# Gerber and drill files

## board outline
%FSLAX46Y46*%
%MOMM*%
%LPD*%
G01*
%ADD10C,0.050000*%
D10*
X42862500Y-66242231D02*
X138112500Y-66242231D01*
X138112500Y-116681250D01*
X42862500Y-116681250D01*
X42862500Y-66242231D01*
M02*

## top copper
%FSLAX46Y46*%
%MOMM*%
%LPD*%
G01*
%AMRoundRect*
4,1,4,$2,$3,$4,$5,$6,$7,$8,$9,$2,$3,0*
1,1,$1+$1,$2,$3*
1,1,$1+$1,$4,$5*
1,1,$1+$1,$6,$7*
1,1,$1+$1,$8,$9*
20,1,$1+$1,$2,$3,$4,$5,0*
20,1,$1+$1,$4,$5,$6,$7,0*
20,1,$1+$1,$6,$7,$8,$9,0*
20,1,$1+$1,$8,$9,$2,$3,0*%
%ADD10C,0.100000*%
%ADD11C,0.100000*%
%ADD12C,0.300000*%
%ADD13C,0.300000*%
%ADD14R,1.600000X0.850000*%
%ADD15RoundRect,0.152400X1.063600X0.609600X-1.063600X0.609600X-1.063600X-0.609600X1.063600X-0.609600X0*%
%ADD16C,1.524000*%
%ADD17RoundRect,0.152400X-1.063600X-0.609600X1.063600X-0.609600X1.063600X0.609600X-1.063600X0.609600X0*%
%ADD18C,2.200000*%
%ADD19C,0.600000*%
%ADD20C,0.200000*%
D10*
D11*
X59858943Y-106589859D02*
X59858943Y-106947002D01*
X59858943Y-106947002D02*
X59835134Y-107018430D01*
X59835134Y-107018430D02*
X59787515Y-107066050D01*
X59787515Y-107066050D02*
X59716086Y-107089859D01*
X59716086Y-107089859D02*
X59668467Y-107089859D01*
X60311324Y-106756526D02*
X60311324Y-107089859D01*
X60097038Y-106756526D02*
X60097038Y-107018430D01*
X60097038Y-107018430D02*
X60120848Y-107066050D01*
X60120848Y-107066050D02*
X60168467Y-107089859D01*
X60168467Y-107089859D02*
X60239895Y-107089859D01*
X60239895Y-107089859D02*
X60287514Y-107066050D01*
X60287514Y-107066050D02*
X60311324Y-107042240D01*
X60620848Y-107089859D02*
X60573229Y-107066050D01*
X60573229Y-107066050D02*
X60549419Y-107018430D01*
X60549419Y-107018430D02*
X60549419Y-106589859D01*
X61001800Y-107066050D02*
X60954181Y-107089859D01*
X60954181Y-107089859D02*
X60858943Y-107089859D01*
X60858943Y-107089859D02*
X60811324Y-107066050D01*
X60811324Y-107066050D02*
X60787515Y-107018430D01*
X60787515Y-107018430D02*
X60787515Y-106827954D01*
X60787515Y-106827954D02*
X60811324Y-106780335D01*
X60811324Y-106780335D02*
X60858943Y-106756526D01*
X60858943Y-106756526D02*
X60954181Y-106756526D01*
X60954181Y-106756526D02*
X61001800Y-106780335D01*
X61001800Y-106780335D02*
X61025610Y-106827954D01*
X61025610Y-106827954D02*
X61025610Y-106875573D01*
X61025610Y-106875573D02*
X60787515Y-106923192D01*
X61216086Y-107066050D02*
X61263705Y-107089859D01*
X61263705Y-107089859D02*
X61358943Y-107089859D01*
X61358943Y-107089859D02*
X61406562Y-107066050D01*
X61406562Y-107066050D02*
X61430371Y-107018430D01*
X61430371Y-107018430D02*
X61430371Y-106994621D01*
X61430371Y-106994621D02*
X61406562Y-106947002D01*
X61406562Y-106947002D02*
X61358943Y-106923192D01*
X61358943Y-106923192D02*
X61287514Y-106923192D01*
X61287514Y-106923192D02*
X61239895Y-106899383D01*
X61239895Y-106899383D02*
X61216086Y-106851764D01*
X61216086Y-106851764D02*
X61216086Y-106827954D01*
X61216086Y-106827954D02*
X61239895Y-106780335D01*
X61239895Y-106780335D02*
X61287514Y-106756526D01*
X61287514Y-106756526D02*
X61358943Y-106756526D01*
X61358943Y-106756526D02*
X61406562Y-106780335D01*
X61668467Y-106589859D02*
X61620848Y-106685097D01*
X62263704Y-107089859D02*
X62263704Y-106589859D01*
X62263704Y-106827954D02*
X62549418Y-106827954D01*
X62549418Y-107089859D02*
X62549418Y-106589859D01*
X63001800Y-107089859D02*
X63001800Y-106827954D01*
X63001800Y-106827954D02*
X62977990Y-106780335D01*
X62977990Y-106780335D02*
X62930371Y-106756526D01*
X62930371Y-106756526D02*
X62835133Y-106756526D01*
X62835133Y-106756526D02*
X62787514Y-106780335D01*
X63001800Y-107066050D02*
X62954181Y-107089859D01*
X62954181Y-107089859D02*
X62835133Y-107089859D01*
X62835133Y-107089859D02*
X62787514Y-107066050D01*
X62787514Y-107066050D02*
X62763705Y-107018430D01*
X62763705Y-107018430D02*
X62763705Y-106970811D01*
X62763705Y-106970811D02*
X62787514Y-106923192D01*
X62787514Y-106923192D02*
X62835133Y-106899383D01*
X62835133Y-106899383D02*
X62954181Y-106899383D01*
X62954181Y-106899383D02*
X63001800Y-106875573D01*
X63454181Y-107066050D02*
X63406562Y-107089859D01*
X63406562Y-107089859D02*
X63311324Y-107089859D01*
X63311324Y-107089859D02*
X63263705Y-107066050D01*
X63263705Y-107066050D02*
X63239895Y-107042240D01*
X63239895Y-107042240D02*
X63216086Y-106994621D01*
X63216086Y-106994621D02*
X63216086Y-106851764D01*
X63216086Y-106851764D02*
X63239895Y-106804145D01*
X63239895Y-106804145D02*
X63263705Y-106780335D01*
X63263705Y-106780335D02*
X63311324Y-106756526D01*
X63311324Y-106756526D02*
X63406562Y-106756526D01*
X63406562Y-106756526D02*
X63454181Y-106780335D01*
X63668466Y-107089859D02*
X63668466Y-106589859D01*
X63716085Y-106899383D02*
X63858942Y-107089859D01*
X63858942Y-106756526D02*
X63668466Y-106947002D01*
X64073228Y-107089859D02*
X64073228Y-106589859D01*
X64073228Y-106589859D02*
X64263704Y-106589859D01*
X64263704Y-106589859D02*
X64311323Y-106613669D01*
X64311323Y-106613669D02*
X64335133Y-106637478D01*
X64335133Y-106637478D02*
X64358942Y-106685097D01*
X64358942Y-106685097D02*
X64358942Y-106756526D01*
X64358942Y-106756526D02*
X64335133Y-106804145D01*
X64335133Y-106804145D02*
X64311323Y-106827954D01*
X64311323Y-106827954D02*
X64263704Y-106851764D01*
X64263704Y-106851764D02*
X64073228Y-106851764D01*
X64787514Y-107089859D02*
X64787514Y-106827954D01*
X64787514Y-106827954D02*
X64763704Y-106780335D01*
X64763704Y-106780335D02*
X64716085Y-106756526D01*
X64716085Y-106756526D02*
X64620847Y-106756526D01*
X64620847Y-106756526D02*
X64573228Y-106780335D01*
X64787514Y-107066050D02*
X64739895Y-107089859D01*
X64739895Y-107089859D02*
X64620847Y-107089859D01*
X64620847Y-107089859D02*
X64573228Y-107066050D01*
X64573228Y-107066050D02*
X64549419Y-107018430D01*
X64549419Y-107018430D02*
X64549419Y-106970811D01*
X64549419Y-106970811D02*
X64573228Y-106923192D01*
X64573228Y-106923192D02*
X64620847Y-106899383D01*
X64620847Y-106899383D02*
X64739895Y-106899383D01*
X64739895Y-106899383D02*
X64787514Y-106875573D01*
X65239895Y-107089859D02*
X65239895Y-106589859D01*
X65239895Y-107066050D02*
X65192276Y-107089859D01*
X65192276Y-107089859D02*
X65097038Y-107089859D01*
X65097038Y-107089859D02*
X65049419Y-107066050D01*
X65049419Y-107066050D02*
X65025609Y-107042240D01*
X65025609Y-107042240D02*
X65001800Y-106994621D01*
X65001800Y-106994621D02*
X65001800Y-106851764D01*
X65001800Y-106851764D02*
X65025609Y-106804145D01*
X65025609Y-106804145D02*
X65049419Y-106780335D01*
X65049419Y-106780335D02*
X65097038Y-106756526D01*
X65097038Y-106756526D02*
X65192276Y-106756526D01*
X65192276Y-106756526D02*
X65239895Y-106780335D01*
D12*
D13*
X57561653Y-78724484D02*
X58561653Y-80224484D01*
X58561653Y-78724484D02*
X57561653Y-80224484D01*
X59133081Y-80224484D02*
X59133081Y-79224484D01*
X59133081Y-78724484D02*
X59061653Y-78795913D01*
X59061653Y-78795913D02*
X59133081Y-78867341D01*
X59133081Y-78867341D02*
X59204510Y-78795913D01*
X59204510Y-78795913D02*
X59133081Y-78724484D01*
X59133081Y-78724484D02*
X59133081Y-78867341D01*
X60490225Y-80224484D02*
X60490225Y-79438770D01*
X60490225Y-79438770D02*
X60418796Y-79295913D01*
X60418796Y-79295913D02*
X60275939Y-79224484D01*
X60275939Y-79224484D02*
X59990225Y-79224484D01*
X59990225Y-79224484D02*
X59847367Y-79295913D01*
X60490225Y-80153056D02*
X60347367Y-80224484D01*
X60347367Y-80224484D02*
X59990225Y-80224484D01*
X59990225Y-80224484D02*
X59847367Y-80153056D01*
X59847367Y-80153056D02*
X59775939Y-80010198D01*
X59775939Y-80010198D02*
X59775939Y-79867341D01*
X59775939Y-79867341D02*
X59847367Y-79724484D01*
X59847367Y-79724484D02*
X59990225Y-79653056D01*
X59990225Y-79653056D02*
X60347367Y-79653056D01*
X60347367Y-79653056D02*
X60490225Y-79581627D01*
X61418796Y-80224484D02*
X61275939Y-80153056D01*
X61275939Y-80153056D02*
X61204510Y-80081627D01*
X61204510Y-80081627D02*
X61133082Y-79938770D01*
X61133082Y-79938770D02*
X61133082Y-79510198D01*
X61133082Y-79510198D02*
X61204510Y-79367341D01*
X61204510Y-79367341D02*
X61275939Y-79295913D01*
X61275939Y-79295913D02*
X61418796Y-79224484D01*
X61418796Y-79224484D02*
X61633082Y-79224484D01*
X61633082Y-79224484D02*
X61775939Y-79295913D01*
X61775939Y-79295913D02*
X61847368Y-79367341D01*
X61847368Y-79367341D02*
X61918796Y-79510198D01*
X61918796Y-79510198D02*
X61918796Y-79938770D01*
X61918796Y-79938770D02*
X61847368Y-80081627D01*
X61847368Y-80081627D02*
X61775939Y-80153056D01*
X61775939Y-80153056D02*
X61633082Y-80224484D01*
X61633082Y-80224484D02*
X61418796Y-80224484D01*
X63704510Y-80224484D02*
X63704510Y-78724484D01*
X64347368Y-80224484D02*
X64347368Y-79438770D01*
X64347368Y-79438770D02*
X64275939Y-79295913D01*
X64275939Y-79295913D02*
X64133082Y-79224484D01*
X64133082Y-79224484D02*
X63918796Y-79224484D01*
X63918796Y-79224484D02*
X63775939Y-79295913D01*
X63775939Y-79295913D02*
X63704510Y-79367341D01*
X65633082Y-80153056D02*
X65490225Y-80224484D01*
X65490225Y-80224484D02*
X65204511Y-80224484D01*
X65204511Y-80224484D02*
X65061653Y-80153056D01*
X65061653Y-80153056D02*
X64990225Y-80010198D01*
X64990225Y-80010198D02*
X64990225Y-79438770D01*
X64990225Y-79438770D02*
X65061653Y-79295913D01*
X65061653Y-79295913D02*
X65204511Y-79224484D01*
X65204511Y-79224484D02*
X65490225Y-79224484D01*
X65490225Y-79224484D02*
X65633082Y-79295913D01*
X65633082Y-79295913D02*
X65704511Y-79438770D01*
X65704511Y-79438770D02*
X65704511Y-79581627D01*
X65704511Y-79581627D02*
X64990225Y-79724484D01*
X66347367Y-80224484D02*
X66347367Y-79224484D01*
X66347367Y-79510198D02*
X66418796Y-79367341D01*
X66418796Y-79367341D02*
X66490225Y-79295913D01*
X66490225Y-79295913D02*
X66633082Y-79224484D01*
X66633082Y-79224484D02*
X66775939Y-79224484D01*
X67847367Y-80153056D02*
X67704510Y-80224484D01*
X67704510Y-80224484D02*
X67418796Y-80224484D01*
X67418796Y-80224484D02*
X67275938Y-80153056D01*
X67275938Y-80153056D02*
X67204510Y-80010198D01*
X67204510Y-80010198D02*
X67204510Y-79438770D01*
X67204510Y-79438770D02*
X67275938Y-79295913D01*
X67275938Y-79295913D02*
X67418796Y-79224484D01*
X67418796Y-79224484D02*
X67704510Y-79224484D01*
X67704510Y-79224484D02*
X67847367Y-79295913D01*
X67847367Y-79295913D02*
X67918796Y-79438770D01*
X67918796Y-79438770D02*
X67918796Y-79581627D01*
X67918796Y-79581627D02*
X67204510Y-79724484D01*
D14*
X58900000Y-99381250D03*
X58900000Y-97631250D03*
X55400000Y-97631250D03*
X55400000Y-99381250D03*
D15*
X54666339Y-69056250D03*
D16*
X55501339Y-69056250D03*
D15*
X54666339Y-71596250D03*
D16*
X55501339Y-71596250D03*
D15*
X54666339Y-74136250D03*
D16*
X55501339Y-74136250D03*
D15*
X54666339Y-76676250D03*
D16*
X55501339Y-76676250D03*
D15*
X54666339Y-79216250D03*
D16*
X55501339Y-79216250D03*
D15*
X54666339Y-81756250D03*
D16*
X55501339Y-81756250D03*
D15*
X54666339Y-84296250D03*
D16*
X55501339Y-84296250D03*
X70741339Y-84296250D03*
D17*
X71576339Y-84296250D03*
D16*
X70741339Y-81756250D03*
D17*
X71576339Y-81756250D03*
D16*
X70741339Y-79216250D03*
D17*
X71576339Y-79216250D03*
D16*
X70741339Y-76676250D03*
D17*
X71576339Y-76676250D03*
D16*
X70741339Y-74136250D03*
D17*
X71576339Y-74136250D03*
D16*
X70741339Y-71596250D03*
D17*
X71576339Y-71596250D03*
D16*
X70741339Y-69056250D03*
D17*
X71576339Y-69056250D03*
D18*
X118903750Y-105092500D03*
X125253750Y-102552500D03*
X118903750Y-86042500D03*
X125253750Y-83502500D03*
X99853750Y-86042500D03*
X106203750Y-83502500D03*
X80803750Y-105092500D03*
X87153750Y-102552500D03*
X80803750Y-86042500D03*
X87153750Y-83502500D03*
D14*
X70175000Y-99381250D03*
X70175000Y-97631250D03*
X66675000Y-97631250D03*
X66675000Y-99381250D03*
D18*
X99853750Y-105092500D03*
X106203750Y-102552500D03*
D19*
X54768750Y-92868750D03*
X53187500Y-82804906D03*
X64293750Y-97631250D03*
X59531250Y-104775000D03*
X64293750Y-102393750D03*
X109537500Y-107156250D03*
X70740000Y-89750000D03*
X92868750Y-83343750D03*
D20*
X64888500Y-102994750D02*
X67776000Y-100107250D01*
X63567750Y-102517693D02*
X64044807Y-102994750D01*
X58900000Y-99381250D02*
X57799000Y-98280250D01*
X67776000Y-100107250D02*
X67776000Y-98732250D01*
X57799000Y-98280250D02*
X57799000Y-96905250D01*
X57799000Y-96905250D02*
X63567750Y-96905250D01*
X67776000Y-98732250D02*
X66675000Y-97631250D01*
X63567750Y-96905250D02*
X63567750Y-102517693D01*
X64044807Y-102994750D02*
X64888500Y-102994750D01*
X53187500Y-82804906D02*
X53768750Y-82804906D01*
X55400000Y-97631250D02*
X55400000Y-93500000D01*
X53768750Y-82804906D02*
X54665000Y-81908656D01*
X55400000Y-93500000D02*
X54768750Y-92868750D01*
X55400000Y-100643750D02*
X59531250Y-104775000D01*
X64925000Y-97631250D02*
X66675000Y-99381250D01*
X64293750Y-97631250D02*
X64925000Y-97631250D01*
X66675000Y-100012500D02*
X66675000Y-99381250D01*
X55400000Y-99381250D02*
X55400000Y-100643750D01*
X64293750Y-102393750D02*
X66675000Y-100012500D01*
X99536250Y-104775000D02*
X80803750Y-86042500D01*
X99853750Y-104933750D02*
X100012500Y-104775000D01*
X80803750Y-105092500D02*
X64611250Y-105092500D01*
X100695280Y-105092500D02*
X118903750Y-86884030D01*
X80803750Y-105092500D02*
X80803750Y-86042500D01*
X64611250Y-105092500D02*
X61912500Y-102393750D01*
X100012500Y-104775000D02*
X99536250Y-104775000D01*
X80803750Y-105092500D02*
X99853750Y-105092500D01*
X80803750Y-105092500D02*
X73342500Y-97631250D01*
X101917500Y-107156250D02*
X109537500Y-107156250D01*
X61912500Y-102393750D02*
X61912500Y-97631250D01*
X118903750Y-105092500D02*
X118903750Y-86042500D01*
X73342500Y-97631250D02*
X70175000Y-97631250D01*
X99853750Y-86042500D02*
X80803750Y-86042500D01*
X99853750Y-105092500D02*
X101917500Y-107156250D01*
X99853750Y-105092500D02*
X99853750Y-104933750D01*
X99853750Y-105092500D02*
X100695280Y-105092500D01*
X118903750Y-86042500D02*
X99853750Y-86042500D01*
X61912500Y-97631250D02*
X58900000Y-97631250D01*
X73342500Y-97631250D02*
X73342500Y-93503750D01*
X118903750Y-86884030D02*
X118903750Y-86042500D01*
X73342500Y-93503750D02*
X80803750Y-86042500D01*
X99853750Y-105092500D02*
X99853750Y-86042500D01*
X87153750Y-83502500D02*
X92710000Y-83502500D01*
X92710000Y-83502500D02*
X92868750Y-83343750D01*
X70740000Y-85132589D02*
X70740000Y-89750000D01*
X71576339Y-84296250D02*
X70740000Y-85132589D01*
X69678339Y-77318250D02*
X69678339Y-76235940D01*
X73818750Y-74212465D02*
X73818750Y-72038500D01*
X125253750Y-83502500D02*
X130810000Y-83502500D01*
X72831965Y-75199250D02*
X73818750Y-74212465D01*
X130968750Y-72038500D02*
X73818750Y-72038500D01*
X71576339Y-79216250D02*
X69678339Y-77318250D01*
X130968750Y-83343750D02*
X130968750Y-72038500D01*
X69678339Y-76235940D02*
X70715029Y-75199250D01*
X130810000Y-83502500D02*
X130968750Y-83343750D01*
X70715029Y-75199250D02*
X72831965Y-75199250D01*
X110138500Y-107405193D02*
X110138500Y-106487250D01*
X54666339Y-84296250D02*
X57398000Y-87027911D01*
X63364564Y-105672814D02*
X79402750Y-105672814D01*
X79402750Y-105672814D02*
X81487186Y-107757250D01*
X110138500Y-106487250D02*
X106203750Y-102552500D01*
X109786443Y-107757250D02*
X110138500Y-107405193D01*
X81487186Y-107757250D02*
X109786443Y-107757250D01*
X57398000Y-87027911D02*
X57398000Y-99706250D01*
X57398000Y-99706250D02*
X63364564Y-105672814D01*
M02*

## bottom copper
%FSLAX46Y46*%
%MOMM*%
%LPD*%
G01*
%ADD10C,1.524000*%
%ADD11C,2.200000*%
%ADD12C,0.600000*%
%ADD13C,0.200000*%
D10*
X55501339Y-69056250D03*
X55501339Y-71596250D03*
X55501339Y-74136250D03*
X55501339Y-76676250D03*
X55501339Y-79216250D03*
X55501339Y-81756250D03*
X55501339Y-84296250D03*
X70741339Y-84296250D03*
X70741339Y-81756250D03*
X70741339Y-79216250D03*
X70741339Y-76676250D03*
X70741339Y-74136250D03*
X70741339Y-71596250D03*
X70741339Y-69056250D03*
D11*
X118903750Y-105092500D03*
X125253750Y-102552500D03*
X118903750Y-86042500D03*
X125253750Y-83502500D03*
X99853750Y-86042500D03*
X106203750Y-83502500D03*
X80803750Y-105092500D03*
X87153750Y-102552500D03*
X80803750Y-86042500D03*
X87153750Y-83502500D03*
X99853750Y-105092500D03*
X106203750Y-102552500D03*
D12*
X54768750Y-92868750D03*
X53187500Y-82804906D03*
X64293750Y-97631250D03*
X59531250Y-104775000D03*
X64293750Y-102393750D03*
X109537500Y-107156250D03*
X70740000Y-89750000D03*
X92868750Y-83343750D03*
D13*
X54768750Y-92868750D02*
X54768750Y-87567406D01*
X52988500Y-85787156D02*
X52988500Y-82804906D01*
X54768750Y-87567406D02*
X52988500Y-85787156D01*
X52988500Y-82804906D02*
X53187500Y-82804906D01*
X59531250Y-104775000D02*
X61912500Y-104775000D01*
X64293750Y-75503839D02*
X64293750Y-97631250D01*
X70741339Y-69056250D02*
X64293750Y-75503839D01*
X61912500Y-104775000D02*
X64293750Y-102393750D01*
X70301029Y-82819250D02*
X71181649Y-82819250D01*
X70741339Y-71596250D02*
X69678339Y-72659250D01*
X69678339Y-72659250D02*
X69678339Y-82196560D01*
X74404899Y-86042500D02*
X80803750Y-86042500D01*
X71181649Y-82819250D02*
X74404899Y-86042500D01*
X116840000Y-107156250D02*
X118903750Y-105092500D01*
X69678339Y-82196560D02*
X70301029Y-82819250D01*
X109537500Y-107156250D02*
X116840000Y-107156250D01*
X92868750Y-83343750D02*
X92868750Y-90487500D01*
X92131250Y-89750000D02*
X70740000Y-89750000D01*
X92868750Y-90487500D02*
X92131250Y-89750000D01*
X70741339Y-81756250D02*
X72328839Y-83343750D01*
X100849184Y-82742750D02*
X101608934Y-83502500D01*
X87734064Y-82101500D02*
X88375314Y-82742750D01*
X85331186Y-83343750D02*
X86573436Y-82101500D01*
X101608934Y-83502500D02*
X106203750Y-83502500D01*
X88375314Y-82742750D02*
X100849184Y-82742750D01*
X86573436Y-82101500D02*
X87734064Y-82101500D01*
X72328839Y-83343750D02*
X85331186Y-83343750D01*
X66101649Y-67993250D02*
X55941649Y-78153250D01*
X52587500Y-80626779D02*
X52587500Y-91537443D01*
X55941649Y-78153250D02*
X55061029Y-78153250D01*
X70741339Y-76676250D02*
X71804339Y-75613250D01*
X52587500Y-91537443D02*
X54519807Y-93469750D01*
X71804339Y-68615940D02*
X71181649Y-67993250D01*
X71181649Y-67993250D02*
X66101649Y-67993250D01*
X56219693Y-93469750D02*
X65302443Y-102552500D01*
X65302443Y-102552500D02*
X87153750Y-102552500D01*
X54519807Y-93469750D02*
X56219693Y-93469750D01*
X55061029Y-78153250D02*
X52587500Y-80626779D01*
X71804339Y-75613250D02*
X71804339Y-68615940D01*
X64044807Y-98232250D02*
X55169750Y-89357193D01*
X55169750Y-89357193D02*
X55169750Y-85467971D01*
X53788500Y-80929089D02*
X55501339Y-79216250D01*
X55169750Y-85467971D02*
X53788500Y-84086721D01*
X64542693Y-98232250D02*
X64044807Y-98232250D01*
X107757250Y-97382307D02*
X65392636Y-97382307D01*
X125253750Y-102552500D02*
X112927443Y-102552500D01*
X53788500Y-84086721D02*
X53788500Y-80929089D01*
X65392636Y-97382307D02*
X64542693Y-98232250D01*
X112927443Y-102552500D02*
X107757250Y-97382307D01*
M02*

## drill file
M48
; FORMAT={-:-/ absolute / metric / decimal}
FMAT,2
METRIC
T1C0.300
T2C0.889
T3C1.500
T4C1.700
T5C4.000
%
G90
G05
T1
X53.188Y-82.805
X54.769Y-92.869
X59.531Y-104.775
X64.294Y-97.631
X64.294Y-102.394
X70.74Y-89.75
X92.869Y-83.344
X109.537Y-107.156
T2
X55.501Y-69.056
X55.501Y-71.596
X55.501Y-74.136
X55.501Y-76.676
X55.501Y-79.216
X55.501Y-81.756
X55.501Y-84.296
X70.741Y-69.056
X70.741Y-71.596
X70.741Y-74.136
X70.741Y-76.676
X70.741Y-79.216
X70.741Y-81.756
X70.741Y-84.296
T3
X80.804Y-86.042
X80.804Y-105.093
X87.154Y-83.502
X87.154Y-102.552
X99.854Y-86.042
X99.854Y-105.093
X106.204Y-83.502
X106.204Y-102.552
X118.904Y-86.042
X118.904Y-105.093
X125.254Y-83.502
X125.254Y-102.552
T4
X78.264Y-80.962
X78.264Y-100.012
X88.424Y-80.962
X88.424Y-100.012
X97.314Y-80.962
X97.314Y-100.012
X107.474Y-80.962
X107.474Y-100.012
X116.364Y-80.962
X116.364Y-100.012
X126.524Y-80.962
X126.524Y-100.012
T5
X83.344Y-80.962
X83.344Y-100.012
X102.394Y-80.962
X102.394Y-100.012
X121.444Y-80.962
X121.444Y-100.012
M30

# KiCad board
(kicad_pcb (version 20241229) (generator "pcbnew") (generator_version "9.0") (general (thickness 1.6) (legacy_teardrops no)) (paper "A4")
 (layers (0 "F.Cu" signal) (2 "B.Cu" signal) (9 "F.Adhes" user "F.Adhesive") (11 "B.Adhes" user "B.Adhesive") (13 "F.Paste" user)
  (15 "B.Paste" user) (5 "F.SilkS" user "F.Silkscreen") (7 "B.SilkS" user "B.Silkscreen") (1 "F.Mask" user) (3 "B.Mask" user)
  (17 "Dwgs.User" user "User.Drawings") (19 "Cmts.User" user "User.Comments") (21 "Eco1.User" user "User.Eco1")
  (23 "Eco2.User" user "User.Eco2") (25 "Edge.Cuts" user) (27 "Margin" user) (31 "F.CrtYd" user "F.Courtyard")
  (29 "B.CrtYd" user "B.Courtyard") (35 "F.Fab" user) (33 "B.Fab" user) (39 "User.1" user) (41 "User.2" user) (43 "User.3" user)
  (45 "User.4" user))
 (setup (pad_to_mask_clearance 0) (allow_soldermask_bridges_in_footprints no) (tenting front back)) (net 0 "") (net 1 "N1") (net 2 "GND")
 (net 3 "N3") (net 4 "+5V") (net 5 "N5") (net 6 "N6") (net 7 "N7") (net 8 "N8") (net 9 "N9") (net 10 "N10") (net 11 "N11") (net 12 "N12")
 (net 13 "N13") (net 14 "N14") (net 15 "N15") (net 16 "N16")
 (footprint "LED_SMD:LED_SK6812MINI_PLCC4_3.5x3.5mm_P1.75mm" (layer "F.Cu") (at 57.15 98.50625 180)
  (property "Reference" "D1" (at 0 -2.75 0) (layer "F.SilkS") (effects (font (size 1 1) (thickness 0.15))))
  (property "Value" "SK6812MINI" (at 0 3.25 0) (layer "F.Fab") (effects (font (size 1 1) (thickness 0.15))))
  (pad "1" smd rect (at -1.75 -0.875 180) (size 1.6 0.85) (layers "F.Cu" "F.Mask" "F.Paste") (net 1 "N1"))
  (pad "2" smd rect (at -1.75 0.875 180) (size 1.6 0.85) (layers "F.Cu" "F.Mask" "F.Paste") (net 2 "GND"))
  (pad "3" smd rect (at 1.75 0.875 180) (size 1.6 0.85) (layers "F.Cu" "F.Mask" "F.Paste") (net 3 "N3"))
  (pad "4" smd rect (at 1.75 -0.875 180) (size 1.6 0.85) (layers "F.Cu" "F.Mask" "F.Paste") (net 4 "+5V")))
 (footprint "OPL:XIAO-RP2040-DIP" (layer "F.Cu") (at 63.121339 76.67625)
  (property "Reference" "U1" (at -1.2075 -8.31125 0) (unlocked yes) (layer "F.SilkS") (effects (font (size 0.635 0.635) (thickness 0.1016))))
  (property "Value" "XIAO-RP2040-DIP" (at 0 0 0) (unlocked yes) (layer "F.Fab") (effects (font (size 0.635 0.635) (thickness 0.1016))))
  (pad "1" smd roundrect (at -8.455 -7.62 180) (size 2.432 1.524) (layers "F.Cu" "F.Mask") (roundrect_rratio 0.1) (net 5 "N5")
   (thermal_bridge_angle 45))
  (pad "1" thru_hole circle (at -7.62 -7.62 180) (size 1.524 1.524) (drill 0.889) (layers "*.Cu" "*.Mask") (remove_unused_layers no)
   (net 5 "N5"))
  (pad "2" smd roundrect (at -8.455 -5.08 180) (size 2.432 1.524) (layers "F.Cu" "F.Mask") (roundrect_rratio 0.1) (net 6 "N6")
   (thermal_bridge_angle 45))
  (pad "2" thru_hole circle (at -7.62 -5.08 180) (size 1.524 1.524) (drill 0.889) (layers "*.Cu" "*.Mask") (remove_unused_layers no)
   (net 6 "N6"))
  (pad "3" smd roundrect (at -8.455 -2.54 180) (size 2.432 1.524) (layers "F.Cu" "F.Mask") (roundrect_rratio 0.1) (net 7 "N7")
   (thermal_bridge_angle 45))
  (pad "3" thru_hole circle (at -7.62 -2.54 180) (size 1.524 1.524) (drill 0.889) (layers "*.Cu" "*.Mask") (remove_unused_layers no)
   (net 7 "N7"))
  (pad "4" smd roundrect (at -8.455 0 180) (size 2.432 1.524) (layers "F.Cu" "F.Mask") (roundrect_rratio 0.1) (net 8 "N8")
   (thermal_bridge_angle 45))
  (pad "4" thru_hole circle (at -7.62 0 180) (size 1.524 1.524) (drill 0.889) (layers "*.Cu" "*.Mask") (remove_unused_layers no)
   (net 8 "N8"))
  (pad "5" smd roundrect (at -8.455 2.54 180) (size 2.432 1.524) (layers "F.Cu" "F.Mask") (roundrect_rratio 0.1) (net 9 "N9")
   (thermal_bridge_angle 45))
  (pad "5" thru_hole circle (at -7.62 2.54 180) (size 1.524 1.524) (drill 0.889) (layers "*.Cu" "*.Mask") (remove_unused_layers no)
   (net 9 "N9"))
  (pad "6" smd roundrect (at -8.455 5.08 180) (size 2.432 1.524) (layers "F.Cu" "F.Mask") (roundrect_rratio 0.1) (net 3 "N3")
   (thermal_bridge_angle 45))
  (pad "6" thru_hole circle (at -7.62 5.08 180) (size 1.524 1.524) (drill 0.889) (layers "*.Cu" "*.Mask") (remove_unused_layers no)
   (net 3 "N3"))
  (pad "7" smd roundrect (at -8.455 7.62 180) (size 2.432 1.524) (layers "F.Cu" "F.Mask") (roundrect_rratio 0.1) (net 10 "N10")
   (thermal_bridge_angle 45))
  (pad "7" thru_hole circle (at -7.62 7.62 180) (size 1.524 1.524) (drill 0.889) (layers "*.Cu" "*.Mask") (remove_unused_layers no)
   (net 10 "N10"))
  (pad "8" thru_hole circle (at 7.62 7.62) (size 1.524 1.524) (drill 0.889) (layers "*.Cu" "*.Mask") (remove_unused_layers no)
   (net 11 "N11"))
  (pad "8" smd roundrect (at 8.455 7.62) (size 2.432 1.524) (layers "F.Cu" "F.Mask") (roundrect_rratio 0.1) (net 11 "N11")
   (thermal_bridge_angle 45))
  (pad "9" thru_hole circle (at 7.62 5.08) (size 1.524 1.524) (drill 0.889) (layers "*.Cu" "*.Mask") (remove_unused_layers no)
   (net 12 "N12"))
  (pad "9" smd roundrect (at 8.455 5.08) (size 2.432 1.524) (layers "F.Cu" "F.Mask") (roundrect_rratio 0.1) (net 12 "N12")
   (thermal_bridge_angle 45))
  (pad "10" thru_hole circle (at 7.62 2.54) (size 1.524 1.524) (drill 0.889) (layers "*.Cu" "*.Mask") (remove_unused_layers no)
   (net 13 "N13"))
  (pad "10" smd roundrect (at 8.455 2.54) (size 2.432 1.524) (layers "F.Cu" "F.Mask") (roundrect_rratio 0.1) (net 13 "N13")
   (thermal_bridge_angle 45))
  (pad "11" thru_hole circle (at 7.62 0) (size 1.524 1.524) (drill 0.889) (layers "*.Cu" "*.Mask") (remove_unused_layers no) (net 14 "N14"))
  (pad "11" smd roundrect (at 8.455 0) (size 2.432 1.524) (layers "F.Cu" "F.Mask") (roundrect_rratio 0.1) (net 14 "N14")
   (thermal_bridge_angle 45))
  (pad "12" thru_hole circle (at 7.62 -2.54) (size 1.524 1.524) (drill 0.889) (layers "*.Cu" "*.Mask") (remove_unused_layers no)
   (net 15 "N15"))
  (pad "12" smd roundrect (at 8.455 -2.54) (size 2.432 1.524) (layers "F.Cu" "F.Mask") (roundrect_rratio 0.1) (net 15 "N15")
   (thermal_bridge_angle 45))
  (pad "13" thru_hole circle (at 7.62 -5.08) (size 1.524 1.524) (drill 0.889) (layers "*.Cu" "*.Mask") (remove_unused_layers no)
   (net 2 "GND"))
  (pad "13" smd roundrect (at 8.455 -5.08) (size 2.432 1.524) (layers "F.Cu" "F.Mask") (roundrect_rratio 0.1) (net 2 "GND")
   (thermal_bridge_angle 45))
  (pad "14" thru_hole circle (at 7.62 -7.62) (size 1.524 1.524) (drill 0.889) (layers "*.Cu" "*.Mask") (remove_unused_layers no)
   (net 4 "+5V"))
  (pad "14" smd roundrect (at 8.455 -7.62) (size 2.432 1.524) (layers "F.Cu" "F.Mask") (roundrect_rratio 0.1) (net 4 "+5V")
   (thermal_bridge_angle 45)))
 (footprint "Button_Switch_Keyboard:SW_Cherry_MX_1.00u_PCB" (layer "F.Cu") (at 118.90375 105.0925 180)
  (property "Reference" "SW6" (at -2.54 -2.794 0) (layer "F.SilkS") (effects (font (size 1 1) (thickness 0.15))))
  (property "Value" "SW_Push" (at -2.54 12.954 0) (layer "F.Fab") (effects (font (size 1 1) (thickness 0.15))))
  (pad "" np_thru_hole circle (at -7.62 5.08 180) (size 1.7 1.7) (drill 1.7) (layers "*.Cu" "*.Mask"))
  (pad "" np_thru_hole circle (at -2.54 5.08 180) (size 4 4) (drill 4) (layers "*.Cu" "*.Mask"))
  (pad "" np_thru_hole circle (at 2.54 5.08 180) (size 1.7 1.7) (drill 1.7) (layers "*.Cu" "*.Mask"))
  (pad "1" thru_hole circle (at 0 0 180) (size 2.2 2.2) (drill 1.5) (layers "*.Cu" "*.Mask") (remove_unused_layers no) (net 2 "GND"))
  (pad "2" thru_hole circle (at -6.35 2.54 180) (size 2.2 2.2) (drill 1.5) (layers "*.Cu" "*.Mask") (remove_unused_layers no) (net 9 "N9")))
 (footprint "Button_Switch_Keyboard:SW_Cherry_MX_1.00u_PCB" (layer "F.Cu") (at 118.90375 86.0425 180)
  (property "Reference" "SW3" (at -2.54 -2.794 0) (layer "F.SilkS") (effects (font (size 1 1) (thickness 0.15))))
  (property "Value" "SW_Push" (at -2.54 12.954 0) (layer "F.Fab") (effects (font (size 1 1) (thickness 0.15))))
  (pad "" np_thru_hole circle (at -7.62 5.08 180) (size 1.7 1.7) (drill 1.7) (layers "*.Cu" "*.Mask"))
  (pad "" np_thru_hole circle (at -2.54 5.08 180) (size 4 4) (drill 4) (layers "*.Cu" "*.Mask"))
  (pad "" np_thru_hole circle (at 2.54 5.08 180) (size 1.7 1.7) (drill 1.7) (layers "*.Cu" "*.Mask"))
  (pad "1" thru_hole circle (at 0 0 180) (size 2.2 2.2) (drill 1.5) (layers "*.Cu" "*.Mask") (remove_unused_layers no) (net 2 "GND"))
  (pad "2" thru_hole circle (at -6.35 2.54 180) (size 2.2 2.2) (drill 1.5) (layers "*.Cu" "*.Mask") (remove_unused_layers no) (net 13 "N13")))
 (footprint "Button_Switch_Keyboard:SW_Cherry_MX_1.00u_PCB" (layer "F.Cu") (at 99.85375 86.0425 180)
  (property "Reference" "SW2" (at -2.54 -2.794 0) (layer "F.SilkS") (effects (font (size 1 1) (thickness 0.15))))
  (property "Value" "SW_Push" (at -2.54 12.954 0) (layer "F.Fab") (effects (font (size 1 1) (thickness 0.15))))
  (pad "" np_thru_hole circle (at -7.62 5.08 180) (size 1.7 1.7) (drill 1.7) (layers "*.Cu" "*.Mask"))
  (pad "" np_thru_hole circle (at -2.54 5.08 180) (size 4 4) (drill 4) (layers "*.Cu" "*.Mask"))
  (pad "" np_thru_hole circle (at 2.54 5.08 180) (size 1.7 1.7) (drill 1.7) (layers "*.Cu" "*.Mask"))
  (pad "1" thru_hole circle (at 0 0 180) (size 2.2 2.2) (drill 1.5) (layers "*.Cu" "*.Mask") (remove_unused_layers no) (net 2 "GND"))
  (pad "2" thru_hole circle (at -6.35 2.54 180) (size 2.2 2.2) (drill 1.5) (layers "*.Cu" "*.Mask") (remove_unused_layers no) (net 12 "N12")))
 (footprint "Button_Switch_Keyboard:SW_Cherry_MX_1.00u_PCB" (layer "F.Cu") (at 80.80375 105.0925 180)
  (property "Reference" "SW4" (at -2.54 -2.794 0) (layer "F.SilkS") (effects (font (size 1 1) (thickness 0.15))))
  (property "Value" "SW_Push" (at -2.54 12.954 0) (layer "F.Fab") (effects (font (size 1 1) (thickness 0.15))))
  (pad "" np_thru_hole circle (at -7.62 5.08 180) (size 1.7 1.7) (drill 1.7) (layers "*.Cu" "*.Mask"))
  (pad "" np_thru_hole circle (at -2.54 5.08 180) (size 4 4) (drill 4) (layers "*.Cu" "*.Mask"))
  (pad "" np_thru_hole circle (at 2.54 5.08 180) (size 1.7 1.7) (drill 1.7) (layers "*.Cu" "*.Mask"))
  (pad "1" thru_hole circle (at 0 0 180) (size 2.2 2.2) (drill 1.5) (layers "*.Cu" "*.Mask") (remove_unused_layers no) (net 2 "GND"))
  (pad "2" thru_hole circle (at -6.35 2.54 180) (size 2.2 2.2) (drill 1.5) (layers "*.Cu" "*.Mask") (remove_unused_layers no) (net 14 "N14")))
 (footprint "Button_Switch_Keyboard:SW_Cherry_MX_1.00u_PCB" (layer "F.Cu") (at 80.80375 86.0425 180)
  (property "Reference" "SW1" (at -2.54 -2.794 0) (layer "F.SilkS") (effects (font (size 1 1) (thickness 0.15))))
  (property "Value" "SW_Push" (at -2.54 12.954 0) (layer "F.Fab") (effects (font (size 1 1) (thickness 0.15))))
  (pad "" np_thru_hole circle (at -7.62 5.08 180) (size 1.7 1.7) (drill 1.7) (layers "*.Cu" "*.Mask"))
  (pad "" np_thru_hole circle (at -2.54 5.08 180) (size 4 4) (drill 4) (layers "*.Cu" "*.Mask"))
  (pad "" np_thru_hole circle (at 2.54 5.08 180) (size 1.7 1.7) (drill 1.7) (layers "*.Cu" "*.Mask"))
  (pad "1" thru_hole circle (at 0 0 180) (size 2.2 2.2) (drill 1.5) (layers "*.Cu" "*.Mask") (remove_unused_layers no) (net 2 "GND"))
  (pad "2" thru_hole circle (at -6.35 2.54 180) (size 2.2 2.2) (drill 1.5) (layers "*.Cu" "*.Mask") (remove_unused_layers no) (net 11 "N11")))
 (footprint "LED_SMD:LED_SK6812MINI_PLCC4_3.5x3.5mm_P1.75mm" (layer "F.Cu") (at 68.425 98.50625 180)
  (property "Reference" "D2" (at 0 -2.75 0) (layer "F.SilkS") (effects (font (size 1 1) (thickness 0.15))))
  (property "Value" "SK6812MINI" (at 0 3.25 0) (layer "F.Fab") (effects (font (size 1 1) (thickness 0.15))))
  (pad "1" smd rect (at -1.75 -0.875 180) (size 1.6 0.85) (layers "F.Cu" "F.Mask" "F.Paste") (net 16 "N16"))
  (pad "2" smd rect (at -1.75 0.875 180) (size 1.6 0.85) (layers "F.Cu" "F.Mask" "F.Paste") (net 2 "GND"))
  (pad "3" smd rect (at 1.75 0.875 180) (size 1.6 0.85) (layers "F.Cu" "F.Mask" "F.Paste") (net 1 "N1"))
  (pad "4" smd rect (at 1.75 -0.875 180) (size 1.6 0.85) (layers "F.Cu" "F.Mask" "F.Paste") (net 4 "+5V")))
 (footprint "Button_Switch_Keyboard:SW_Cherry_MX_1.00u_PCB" (layer "F.Cu") (at 99.85375 105.0925 180)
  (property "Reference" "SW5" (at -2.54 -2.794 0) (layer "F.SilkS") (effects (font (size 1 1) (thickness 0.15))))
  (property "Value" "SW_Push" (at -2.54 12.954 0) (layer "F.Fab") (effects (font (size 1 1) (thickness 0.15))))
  (pad "" np_thru_hole circle (at -7.62 5.08 180) (size 1.7 1.7) (drill 1.7) (layers "*.Cu" "*.Mask"))
  (pad "" np_thru_hole circle (at -2.54 5.08 180) (size 4 4) (drill 4) (layers "*.Cu" "*.Mask"))
  (pad "" np_thru_hole circle (at 2.54 5.08 180) (size 1.7 1.7) (drill 1.7) (layers "*.Cu" "*.Mask"))
  (pad "1" thru_hole circle (at 0 0 180) (size 2.2 2.2) (drill 1.5) (layers "*.Cu" "*.Mask") (remove_unused_layers no) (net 2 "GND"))
  (pad "2" thru_hole circle (at -6.35 2.54 180) (size 2.2 2.2) (drill 1.5) (layers "*.Cu" "*.Mask") (remove_unused_layers no) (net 10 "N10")))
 (gr_rect (start 42.8625 66.242231) (end 138.1125 116.68125) (stroke (width 0.05) (type default)) (fill no) (layer "Edge.Cuts"))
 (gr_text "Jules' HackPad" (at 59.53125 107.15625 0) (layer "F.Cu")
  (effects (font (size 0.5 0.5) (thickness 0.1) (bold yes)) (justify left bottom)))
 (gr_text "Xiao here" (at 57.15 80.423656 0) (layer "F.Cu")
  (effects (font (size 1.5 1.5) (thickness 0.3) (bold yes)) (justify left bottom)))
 (segment (start 64.8885 102.99475) (end 67.776 100.10725) (width 0.2) (layer "F.Cu") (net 1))
 (segment (start 63.56775 102.517693) (end 64.044807 102.99475) (width 0.2) (layer "F.Cu") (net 1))
 (segment (start 58.9 99.38125) (end 57.799 98.28025) (width 0.2) (layer "F.Cu") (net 1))
 (segment (start 67.776 100.10725) (end 67.776 98.73225) (width 0.2) (layer "F.Cu") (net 1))
 (segment (start 57.799 98.28025) (end 57.799 96.90525) (width 0.2) (layer "F.Cu") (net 1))
 (segment (start 57.799 96.90525) (end 63.56775 96.90525) (width 0.2) (layer "F.Cu") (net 1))
 (segment (start 67.776 98.73225) (end 66.675 97.63125) (width 0.2) (layer "F.Cu") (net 1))
 (segment (start 63.56775 96.90525) (end 63.56775 102.517693) (width 0.2) (layer "F.Cu") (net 1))
 (segment (start 64.044807 102.99475) (end 64.8885 102.99475) (width 0.2) (layer "F.Cu") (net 1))
 (segment (start 53.1875 82.804906) (end 53.76875 82.804906) (width 0.2) (layer "F.Cu") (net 3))
 (segment (start 55.4 97.63125) (end 55.4 93.5) (width 0.2) (layer "F.Cu") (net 3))
 (segment (start 53.76875 82.804906) (end 54.665 81.908656) (width 0.2) (layer "F.Cu") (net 3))
 (segment (start 55.4 93.5) (end 54.76875 92.86875) (width 0.2) (layer "F.Cu") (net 3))
 (via (at 54.76875 92.86875) (size 0.6) (drill 0.3) (layers "F.Cu" "B.Cu") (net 3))
 (via (at 53.1875 82.804906) (size 0.6) (drill 0.3) (layers "F.Cu" "B.Cu") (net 3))
 (segment (start 54.76875 92.86875) (end 54.76875 87.567406) (width 0.2) (layer "B.Cu") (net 3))
 (segment (start 52.9885 85.787156) (end 52.9885 82.804906) (width 0.2) (layer "B.Cu") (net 3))
 (segment (start 54.76875 87.567406) (end 52.9885 85.787156) (width 0.2) (layer "B.Cu") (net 3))
 (segment (start 52.9885 82.804906) (end 53.1875 82.804906) (width 0.2) (layer "B.Cu") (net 3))
 (segment (start 55.4 100.64375) (end 59.53125 104.775) (width 0.2) (layer "F.Cu") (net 4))
 (segment (start 64.925 97.63125) (end 66.675 99.38125) (width 0.2) (layer "F.Cu") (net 4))
 (segment (start 64.29375 97.63125) (end 64.925 97.63125) (width 0.2) (layer "F.Cu") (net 4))
 (segment (start 66.675 100.0125) (end 66.675 99.38125) (width 0.2) (layer "F.Cu") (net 4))
 (segment (start 55.4 99.38125) (end 55.4 100.64375) (width 0.2) (layer "F.Cu") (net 4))
 (segment (start 64.29375 102.39375) (end 66.675 100.0125) (width 0.2) (layer "F.Cu") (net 4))
 (via (at 64.29375 97.63125) (size 0.6) (drill 0.3) (layers "F.Cu" "B.Cu") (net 4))
 (via (at 59.53125 104.775) (size 0.6) (drill 0.3) (layers "F.Cu" "B.Cu") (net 4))
 (via (at 64.29375 102.39375) (size 0.6) (drill 0.3) (layers "F.Cu" "B.Cu") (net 4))
 (segment (start 59.53125 104.775) (end 61.9125 104.775) (width 0.2) (layer "B.Cu") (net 4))
 (segment (start 64.29375 75.503839) (end 64.29375 97.63125) (width 0.2) (layer "B.Cu") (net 4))
 (segment (start 70.741339 69.05625) (end 64.29375 75.503839) (width 0.2) (layer "B.Cu") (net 4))
 (segment (start 61.9125 104.775) (end 64.29375 102.39375) (width 0.2) (layer "B.Cu") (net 4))
 (segment (start 99.53625 104.775) (end 80.80375 86.0425) (width 0.2) (layer "F.Cu") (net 2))
 (segment (start 99.85375 104.93375) (end 100.0125 104.775) (width 0.2) (layer "F.Cu") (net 2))
 (segment (start 80.80375 105.0925) (end 64.61125 105.0925) (width 0.2) (layer "F.Cu") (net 2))
 (segment (start 100.69528 105.0925) (end 118.90375 86.88403) (width 0.2) (layer "F.Cu") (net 2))
 (segment (start 80.80375 105.0925) (end 80.80375 86.0425) (width 0.2) (layer "F.Cu") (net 2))
 (segment (start 64.61125 105.0925) (end 61.9125 102.39375) (width 0.2) (layer "F.Cu") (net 2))
 (segment (start 100.0125 104.775) (end 99.53625 104.775) (width 0.2) (layer "F.Cu") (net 2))
 (segment (start 80.80375 105.0925) (end 99.85375 105.0925) (width 0.2) (layer "F.Cu") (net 2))
 (segment (start 80.80375 105.0925) (end 73.3425 97.63125) (width 0.2) (layer "F.Cu") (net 2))
 (segment (start 101.9175 107.15625) (end 109.5375 107.15625) (width 0.2) (layer "F.Cu") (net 2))
 (segment (start 61.9125 102.39375) (end 61.9125 97.63125) (width 0.2) (layer "F.Cu") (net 2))
 (segment (start 118.90375 105.0925) (end 118.90375 86.0425) (width 0.2) (layer "F.Cu") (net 2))
 (segment (start 73.3425 97.63125) (end 70.175 97.63125) (width 0.2) (layer "F.Cu") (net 2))
 (segment (start 99.85375 86.0425) (end 80.80375 86.0425) (width 0.2) (layer "F.Cu") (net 2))
 (segment (start 99.85375 105.0925) (end 101.9175 107.15625) (width 0.2) (layer "F.Cu") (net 2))
 (segment (start 99.85375 105.0925) (end 99.85375 104.93375) (width 0.2) (layer "F.Cu") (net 2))
 (segment (start 99.85375 105.0925) (end 100.69528 105.0925) (width 0.2) (layer "F.Cu") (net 2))
 (segment (start 118.90375 86.0425) (end 99.85375 86.0425) (width 0.2) (layer "F.Cu") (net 2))
 (segment (start 61.9125 97.63125) (end 58.9 97.63125) (width 0.2) (layer "F.Cu") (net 2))
 (segment (start 73.3425 97.63125) (end 73.3425 93.50375) (width 0.2) (layer "F.Cu") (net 2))
 (segment (start 118.90375 86.88403) (end 118.90375 86.0425) (width 0.2) (layer "F.Cu") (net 2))
 (segment (start 73.3425 93.50375) (end 80.80375 86.0425) (width 0.2) (layer "F.Cu") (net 2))
 (segment (start 99.85375 105.0925) (end 99.85375 86.0425) (width 0.2) (layer "F.Cu") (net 2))
 (via (at 109.5375 107.15625) (size 0.6) (drill 0.3) (layers "F.Cu" "B.Cu") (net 2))
 (segment (start 70.301029 82.81925) (end 71.181649 82.81925) (width 0.2) (layer "B.Cu") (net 2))
 (segment (start 70.741339 71.59625) (end 69.678339 72.65925) (width 0.2) (layer "B.Cu") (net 2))
 (segment (start 69.678339 72.65925) (end 69.678339 82.19656) (width 0.2) (layer "B.Cu") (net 2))
 (segment (start 74.404899 86.0425) (end 80.80375 86.0425) (width 0.2) (layer "B.Cu") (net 2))
 (segment (start 71.181649 82.81925) (end 74.404899 86.0425) (width 0.2) (layer "B.Cu") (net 2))
 (segment (start 116.84 107.15625) (end 118.90375 105.0925) (width 0.2) (layer "B.Cu") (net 2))
 (segment (start 69.678339 82.19656) (end 70.301029 82.81925) (width 0.2) (layer "B.Cu") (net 2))
 (segment (start 109.5375 107.15625) (end 116.84 107.15625) (width 0.2) (layer "B.Cu") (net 2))
 (segment (start 87.15375 83.5025) (end 92.71 83.5025) (width 0.2) (layer "F.Cu") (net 11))
 (segment (start 92.71 83.5025) (end 92.86875 83.34375) (width 0.2) (layer "F.Cu") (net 11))
 (segment (start 70.74 85.132589) (end 70.74 89.75) (width 0.2) (layer "F.Cu") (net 11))
 (segment (start 71.576339 84.29625) (end 70.74 85.132589) (width 0.2) (layer "F.Cu") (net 11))
 (via (at 70.74 89.75) (size 0.6) (drill 0.3) (layers "F.Cu" "B.Cu") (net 11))
 (via (at 92.86875 83.34375) (size 0.6) (drill 0.3) (layers "F.Cu" "B.Cu") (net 11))
 (segment (start 92.86875 83.34375) (end 92.86875 90.4875) (width 0.2) (layer "B.Cu") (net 11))
 (segment (start 92.13125 89.75) (end 70.74 89.75) (width 0.2) (layer "B.Cu") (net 11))
 (segment (start 92.86875 90.4875) (end 92.13125 89.75) (width 0.2) (layer "B.Cu") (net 11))
 (segment (start 70.741339 81.75625) (end 72.328839 83.34375) (width 0.2) (layer "B.Cu") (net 12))
 (segment (start 100.849184 82.74275) (end 101.608934 83.5025) (width 0.2) (layer "B.Cu") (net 12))
 (segment (start 87.734064 82.1015) (end 88.375314 82.74275) (width 0.2) (layer "B.Cu") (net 12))
 (segment (start 85.331186 83.34375) (end 86.573436 82.1015) (width 0.2) (layer "B.Cu") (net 12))
 (segment (start 101.608934 83.5025) (end 106.20375 83.5025) (width 0.2) (layer "B.Cu") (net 12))
 (segment (start 88.375314 82.74275) (end 100.849184 82.74275) (width 0.2) (layer "B.Cu") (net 12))
 (segment (start 86.573436 82.1015) (end 87.734064 82.1015) (width 0.2) (layer "B.Cu") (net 12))
 (segment (start 72.328839 83.34375) (end 85.331186 83.34375) (width 0.2) (layer "B.Cu") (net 12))
 (segment (start 69.678339 77.31825) (end 69.678339 76.23594) (width 0.2) (layer "F.Cu") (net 13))
 (segment (start 73.81875 74.212465) (end 73.81875 72.0385) (width 0.2) (layer "F.Cu") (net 13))
 (segment (start 125.25375 83.5025) (end 130.81 83.5025) (width 0.2) (layer "F.Cu") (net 13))
 (segment (start 72.831965 75.19925) (end 73.81875 74.212465) (width 0.2) (layer "F.Cu") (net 13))
 (segment (start 130.96875 72.0385) (end 73.81875 72.0385) (width 0.2) (layer "F.Cu") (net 13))
 (segment (start 71.576339 79.21625) (end 69.678339 77.31825) (width 0.2) (layer "F.Cu") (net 13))
 (segment (start 130.96875 83.34375) (end 130.96875 72.0385) (width 0.2) (layer "F.Cu") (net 13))
 (segment (start 69.678339 76.23594) (end 70.715029 75.19925) (width 0.2) (layer "F.Cu") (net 13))
 (segment (start 130.81 83.5025) (end 130.96875 83.34375) (width 0.2) (layer "F.Cu") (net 13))
 (segment (start 70.715029 75.19925) (end 72.831965 75.19925) (width 0.2) (layer "F.Cu") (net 13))
 (segment (start 66.101649 67.99325) (end 55.941649 78.15325) (width 0.2) (layer "B.Cu") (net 14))
 (segment (start 52.5875 80.626779) (end 52.5875 91.537443) (width 0.2) (layer "B.Cu") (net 14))
 (segment (start 55.941649 78.15325) (end 55.061029 78.15325) (width 0.2) (layer "B.Cu") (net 14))
 (segment (start 70.741339 76.67625) (end 71.804339 75.61325) (width 0.2) (layer "B.Cu") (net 14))
 (segment (start 52.5875 91.537443) (end 54.519807 93.46975) (width 0.2) (layer "B.Cu") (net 14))
 (segment (start 71.804339 68.61594) (end 71.181649 67.99325) (width 0.2) (layer "B.Cu") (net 14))
 (segment (start 71.181649 67.99325) (end 66.101649 67.99325) (width 0.2) (layer "B.Cu") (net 14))
 (segment (start 56.219693 93.46975) (end 65.302443 102.5525) (width 0.2) (layer "B.Cu") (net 14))
 (segment (start 65.302443 102.5525) (end 87.15375 102.5525) (width 0.2) (layer "B.Cu") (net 14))
 (segment (start 54.519807 93.46975) (end 56.219693 93.46975) (width 0.2) (layer "B.Cu") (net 14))
 (segment (start 55.061029 78.15325) (end 52.5875 80.626779) (width 0.2) (layer "B.Cu") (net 14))
 (segment (start 71.804339 75.61325) (end 71.804339 68.61594) (width 0.2) (layer "B.Cu") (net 14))
 (segment (start 110.1385 107.405193) (end 110.1385 106.48725) (width 0.2) (layer "F.Cu") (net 10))
 (segment (start 54.666339 84.29625) (end 57.398 87.027911) (width 0.2) (layer "F.Cu") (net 10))
 (segment (start 63.364564 105.672814) (end 79.40275 105.672814) (width 0.2) (layer "F.Cu") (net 10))
 (segment (start 79.40275 105.672814) (end 81.487186 107.75725) (width 0.2) (layer "F.Cu") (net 10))
 (segment (start 110.1385 106.48725) (end 106.20375 102.5525) (width 0.2) (layer "F.Cu") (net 10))
 (segment (start 109.786443 107.75725) (end 110.1385 107.405193) (width 0.2) (layer "F.Cu") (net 10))
 (segment (start 81.487186 107.75725) (end 109.786443 107.75725) (width 0.2) (layer "F.Cu") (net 10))
 (segment (start 57.398 87.027911) (end 57.398 99.70625) (width 0.2) (layer "F.Cu") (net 10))
 (segment (start 57.398 99.70625) (end 63.364564 105.672814) (width 0.2) (layer "F.Cu") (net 10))
 (segment (start 64.044807 98.23225) (end 55.16975 89.357193) (width 0.2) (layer "B.Cu") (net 9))
 (segment (start 55.16975 89.357193) (end 55.16975 85.467971) (width 0.2) (layer "B.Cu") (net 9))
 (segment (start 53.7885 80.929089) (end 55.501339 79.21625) (width 0.2) (layer "B.Cu") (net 9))
 (segment (start 55.16975 85.467971) (end 53.7885 84.086721) (width 0.2) (layer "B.Cu") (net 9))
 (segment (start 64.542693 98.23225) (end 64.044807 98.23225) (width 0.2) (layer "B.Cu") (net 9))
 (segment (start 107.75725 97.382307) (end 65.392636 97.382307) (width 0.2) (layer "B.Cu") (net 9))
 (segment (start 125.25375 102.5525) (end 112.927443 102.5525) (width 0.2) (layer "B.Cu") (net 9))
 (segment (start 53.7885 84.086721) (end 53.7885 80.929089) (width 0.2) (layer "B.Cu") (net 9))
 (segment (start 65.392636 97.382307) (end 64.542693 98.23225) (width 0.2) (layer "B.Cu") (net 9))
 (segment (start 112.927443 102.5525) (end 107.75725 97.382307) (width 0.2) (layer "B.Cu") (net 9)))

